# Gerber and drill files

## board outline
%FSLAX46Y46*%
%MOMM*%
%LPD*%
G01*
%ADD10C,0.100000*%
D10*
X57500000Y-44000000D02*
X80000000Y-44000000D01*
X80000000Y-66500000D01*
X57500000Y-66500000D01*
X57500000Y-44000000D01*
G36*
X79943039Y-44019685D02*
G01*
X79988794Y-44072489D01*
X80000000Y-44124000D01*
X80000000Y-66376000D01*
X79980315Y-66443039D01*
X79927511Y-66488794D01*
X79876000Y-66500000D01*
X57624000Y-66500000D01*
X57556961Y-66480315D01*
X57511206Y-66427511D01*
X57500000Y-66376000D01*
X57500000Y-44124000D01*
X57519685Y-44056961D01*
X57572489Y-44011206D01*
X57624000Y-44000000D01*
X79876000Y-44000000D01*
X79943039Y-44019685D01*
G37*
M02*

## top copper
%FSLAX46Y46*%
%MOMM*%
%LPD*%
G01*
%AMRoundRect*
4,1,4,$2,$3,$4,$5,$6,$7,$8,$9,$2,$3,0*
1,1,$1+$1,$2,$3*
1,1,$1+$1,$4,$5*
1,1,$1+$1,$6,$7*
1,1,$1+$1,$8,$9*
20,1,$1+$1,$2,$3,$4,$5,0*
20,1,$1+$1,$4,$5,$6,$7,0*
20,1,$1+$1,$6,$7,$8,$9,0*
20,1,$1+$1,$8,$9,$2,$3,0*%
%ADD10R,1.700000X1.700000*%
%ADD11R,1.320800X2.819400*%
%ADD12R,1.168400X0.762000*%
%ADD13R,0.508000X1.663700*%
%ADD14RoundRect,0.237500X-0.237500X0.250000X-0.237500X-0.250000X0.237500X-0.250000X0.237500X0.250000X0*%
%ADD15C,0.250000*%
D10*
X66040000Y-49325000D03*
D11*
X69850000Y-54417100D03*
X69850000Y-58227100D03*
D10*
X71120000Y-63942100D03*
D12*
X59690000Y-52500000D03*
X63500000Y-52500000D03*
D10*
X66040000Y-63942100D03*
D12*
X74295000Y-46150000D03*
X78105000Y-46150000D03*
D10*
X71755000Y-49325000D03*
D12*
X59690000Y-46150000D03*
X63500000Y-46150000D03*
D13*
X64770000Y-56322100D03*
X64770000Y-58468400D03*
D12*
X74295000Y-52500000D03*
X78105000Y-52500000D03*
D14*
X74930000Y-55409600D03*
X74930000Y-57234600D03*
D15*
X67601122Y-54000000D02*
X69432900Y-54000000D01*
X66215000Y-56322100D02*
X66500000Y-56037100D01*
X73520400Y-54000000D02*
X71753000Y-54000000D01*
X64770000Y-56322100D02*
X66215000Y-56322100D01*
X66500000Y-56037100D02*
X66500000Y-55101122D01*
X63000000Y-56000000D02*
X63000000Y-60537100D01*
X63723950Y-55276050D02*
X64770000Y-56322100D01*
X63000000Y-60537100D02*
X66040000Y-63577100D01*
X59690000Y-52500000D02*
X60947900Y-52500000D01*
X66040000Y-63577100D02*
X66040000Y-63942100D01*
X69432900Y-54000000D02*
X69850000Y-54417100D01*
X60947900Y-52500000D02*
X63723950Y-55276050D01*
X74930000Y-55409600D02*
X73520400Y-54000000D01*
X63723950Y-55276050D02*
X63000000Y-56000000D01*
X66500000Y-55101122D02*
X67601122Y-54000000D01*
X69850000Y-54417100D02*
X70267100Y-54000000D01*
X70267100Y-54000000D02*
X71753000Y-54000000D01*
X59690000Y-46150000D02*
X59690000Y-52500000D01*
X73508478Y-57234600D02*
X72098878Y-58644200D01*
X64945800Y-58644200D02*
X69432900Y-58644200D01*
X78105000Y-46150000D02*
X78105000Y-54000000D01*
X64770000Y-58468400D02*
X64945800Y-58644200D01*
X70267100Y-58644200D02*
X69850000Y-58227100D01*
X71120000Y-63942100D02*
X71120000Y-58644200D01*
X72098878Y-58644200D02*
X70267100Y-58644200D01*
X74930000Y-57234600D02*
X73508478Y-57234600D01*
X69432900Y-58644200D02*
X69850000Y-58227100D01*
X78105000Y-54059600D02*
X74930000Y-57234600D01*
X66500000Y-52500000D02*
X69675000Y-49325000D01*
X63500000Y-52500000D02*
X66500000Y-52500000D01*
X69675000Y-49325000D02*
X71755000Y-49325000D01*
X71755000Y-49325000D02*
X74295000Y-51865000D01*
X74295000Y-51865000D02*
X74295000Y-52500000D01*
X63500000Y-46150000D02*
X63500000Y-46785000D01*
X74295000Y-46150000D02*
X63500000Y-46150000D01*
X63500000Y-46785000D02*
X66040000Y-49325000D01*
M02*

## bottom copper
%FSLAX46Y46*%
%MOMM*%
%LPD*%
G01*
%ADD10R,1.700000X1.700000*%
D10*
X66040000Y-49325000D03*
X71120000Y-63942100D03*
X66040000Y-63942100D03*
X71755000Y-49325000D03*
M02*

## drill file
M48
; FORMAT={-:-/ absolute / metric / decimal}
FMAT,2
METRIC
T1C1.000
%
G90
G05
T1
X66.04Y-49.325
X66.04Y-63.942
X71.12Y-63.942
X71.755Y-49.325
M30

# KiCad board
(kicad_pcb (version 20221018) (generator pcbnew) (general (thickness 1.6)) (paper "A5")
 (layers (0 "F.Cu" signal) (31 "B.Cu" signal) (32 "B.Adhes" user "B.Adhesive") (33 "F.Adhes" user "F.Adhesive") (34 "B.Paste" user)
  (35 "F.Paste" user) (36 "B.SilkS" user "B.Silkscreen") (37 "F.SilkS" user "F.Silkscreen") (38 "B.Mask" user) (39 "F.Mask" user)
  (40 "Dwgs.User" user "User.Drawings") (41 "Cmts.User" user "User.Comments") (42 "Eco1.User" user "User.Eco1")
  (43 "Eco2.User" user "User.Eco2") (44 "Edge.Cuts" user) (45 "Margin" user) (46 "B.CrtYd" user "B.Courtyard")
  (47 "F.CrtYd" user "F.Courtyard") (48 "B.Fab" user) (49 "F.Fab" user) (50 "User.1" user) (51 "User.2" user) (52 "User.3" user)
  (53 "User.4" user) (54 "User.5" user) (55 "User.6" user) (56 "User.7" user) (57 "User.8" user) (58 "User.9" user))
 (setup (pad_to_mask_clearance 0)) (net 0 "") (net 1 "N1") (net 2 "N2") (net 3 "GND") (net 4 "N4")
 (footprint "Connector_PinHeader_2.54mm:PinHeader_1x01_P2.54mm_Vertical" (layer "F.Cu") (at 66.04 49.325)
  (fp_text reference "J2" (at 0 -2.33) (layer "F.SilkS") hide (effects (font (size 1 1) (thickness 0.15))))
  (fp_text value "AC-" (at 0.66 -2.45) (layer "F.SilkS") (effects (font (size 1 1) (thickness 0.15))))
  (pad "1" thru_hole rect (at 0 0) (size 1.7 1.7) (drill 1) (layers "*.Cu" "*.Mask") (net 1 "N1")))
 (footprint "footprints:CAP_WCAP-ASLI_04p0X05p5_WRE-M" (layer "F.Cu") (at 69.85 56.3221 -90)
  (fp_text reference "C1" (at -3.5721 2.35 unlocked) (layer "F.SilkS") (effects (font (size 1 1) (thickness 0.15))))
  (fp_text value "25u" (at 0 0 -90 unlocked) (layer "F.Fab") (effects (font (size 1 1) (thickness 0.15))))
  (pad "1" smd rect (at -1.905 0 270) (size 2.8194 1.3208) (layers "F.Cu" "F.Paste" "F.Mask") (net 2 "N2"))
  (pad "2" smd rect (at 1.905 0 270) (size 2.8194 1.3208) (layers "F.Cu" "F.Paste" "F.Mask") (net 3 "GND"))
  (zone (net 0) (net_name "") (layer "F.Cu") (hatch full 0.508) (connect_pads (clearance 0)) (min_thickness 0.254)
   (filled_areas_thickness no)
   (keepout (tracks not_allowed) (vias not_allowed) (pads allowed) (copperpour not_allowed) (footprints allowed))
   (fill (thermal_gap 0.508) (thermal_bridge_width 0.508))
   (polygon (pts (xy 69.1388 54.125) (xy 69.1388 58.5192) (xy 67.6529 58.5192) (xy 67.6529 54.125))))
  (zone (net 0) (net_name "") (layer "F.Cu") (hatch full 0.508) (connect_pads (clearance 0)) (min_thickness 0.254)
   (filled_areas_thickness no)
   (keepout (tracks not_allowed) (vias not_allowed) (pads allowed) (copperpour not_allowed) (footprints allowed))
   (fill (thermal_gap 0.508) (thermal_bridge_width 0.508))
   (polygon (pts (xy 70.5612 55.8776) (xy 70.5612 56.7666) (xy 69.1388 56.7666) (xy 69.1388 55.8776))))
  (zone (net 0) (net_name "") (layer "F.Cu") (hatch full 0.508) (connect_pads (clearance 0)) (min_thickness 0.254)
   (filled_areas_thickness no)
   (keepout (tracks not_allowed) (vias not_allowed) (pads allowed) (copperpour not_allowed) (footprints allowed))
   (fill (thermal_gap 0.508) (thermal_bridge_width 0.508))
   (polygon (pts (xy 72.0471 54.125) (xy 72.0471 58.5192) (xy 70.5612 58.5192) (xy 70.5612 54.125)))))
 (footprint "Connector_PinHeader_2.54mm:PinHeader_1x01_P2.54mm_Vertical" (layer "F.Cu") (at 71.12 63.9421 90)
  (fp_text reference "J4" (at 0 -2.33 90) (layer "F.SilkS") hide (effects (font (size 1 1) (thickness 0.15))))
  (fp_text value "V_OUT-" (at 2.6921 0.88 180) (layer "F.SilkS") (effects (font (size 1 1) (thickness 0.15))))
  (pad "1" thru_hole rect (at 0 0 90) (size 1.7 1.7) (drill 1) (layers "*.Cu" "*.Mask") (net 3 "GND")))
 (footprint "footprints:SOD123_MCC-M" (layer "F.Cu") (at 61.595 52.5)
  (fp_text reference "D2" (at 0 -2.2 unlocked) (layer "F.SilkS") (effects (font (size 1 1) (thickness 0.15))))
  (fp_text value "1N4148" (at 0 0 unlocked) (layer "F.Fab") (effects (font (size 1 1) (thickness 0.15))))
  (pad "1" smd rect (at -1.905 0) (size 1.1684 0.762) (layers "F.Cu" "F.Paste" "F.Mask") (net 2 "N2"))
  (pad "2" smd rect (at 1.905 0) (size 1.1684 0.762) (layers "F.Cu" "F.Paste" "F.Mask") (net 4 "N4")))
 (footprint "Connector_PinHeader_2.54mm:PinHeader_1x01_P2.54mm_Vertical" (layer "F.Cu") (at 66.04 63.9421 180)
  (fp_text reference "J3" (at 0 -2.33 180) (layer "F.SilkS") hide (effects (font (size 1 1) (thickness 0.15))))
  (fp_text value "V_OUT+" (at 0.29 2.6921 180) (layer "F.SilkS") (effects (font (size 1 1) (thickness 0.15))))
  (pad "1" thru_hole rect (at 0 0 180) (size 1.7 1.7) (drill 1) (layers "*.Cu" "*.Mask") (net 2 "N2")))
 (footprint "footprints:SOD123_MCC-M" (layer "F.Cu") (at 76.2 46.15)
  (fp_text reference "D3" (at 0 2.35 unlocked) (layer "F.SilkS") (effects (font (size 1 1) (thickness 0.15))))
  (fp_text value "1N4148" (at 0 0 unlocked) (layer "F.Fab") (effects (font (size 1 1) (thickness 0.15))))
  (pad "1" smd rect (at -1.905 0) (size 1.1684 0.762) (layers "F.Cu" "F.Paste" "F.Mask") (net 1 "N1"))
  (pad "2" smd rect (at 1.905 0) (size 1.1684 0.762) (layers "F.Cu" "F.Paste" "F.Mask") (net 3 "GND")))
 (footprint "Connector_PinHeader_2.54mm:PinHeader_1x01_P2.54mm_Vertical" (layer "F.Cu") (at 71.755 49.325)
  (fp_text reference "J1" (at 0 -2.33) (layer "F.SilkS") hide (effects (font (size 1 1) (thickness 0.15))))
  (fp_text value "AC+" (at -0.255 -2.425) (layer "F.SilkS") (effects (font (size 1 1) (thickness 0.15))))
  (pad "1" thru_hole rect (at 0 0) (size 1.7 1.7) (drill 1) (layers "*.Cu" "*.Mask") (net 4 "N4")))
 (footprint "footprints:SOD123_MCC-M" (layer "F.Cu") (at 61.595 46.15)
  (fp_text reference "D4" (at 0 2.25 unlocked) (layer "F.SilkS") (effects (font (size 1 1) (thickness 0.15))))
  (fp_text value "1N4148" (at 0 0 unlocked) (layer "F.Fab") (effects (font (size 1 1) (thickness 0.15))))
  (pad "1" smd rect (at -1.905 0) (size 1.1684 0.762) (layers "F.Cu" "F.Paste" "F.Mask") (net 2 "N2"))
  (pad "2" smd rect (at 1.905 0) (size 1.1684 0.762) (layers "F.Cu" "F.Paste" "F.Mask") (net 1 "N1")))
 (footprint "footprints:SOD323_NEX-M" (layer "F.Cu") (at 64.77 57.39525 -90)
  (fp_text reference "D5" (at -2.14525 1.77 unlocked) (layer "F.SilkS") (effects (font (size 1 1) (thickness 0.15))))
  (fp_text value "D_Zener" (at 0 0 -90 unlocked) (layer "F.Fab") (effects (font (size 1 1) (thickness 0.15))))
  (pad "1" smd rect (at -1.07315 0 270) (size 1.6637 0.508) (layers "F.Cu" "F.Paste" "F.Mask") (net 2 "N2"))
  (pad "2" smd rect (at 1.07315 0 270) (size 1.6637 0.508) (layers "F.Cu" "F.Paste" "F.Mask") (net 3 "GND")))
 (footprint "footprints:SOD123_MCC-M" (layer "F.Cu") (at 76.2 52.5)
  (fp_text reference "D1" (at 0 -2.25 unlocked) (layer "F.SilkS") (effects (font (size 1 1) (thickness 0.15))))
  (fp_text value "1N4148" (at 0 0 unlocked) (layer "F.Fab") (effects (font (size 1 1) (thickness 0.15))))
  (pad "1" smd rect (at -1.905 0) (size 1.1684 0.762) (layers "F.Cu" "F.Paste" "F.Mask") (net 4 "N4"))
  (pad "2" smd rect (at 1.905 0) (size 1.1684 0.762) (layers "F.Cu" "F.Paste" "F.Mask") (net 3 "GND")))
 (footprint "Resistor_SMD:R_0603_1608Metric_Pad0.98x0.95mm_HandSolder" (layer "F.Cu") (at 74.93 56.3221 -90)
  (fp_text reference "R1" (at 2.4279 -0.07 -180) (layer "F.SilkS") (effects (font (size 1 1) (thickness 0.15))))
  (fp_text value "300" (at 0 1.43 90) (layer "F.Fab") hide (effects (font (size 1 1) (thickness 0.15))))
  (pad "1" smd roundrect (at -0.9125 0 270) (size 0.975 0.95) (layers "F.Cu" "F.Paste" "F.Mask") (roundrect_rratio 0.25) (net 2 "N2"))
  (pad "2" smd roundrect (at 0.9125 0 270) (size 0.975 0.95) (layers "F.Cu" "F.Paste" "F.Mask") (roundrect_rratio 0.25) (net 3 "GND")))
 (gr_rect (start 57.5 44) (end 80 66.5) (stroke (width 0.1) (type default)) (fill none) (layer "Edge.Cuts"))
 (segment (start 67.601122 54) (end 69.4329 54) (width 0.25) (layer "F.Cu") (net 2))
 (segment (start 66.215 56.3221) (end 66.5 56.0371) (width 0.25) (layer "F.Cu") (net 2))
 (segment (start 73.5204 54) (end 71.753 54) (width 0.25) (layer "F.Cu") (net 2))
 (segment (start 64.77 56.3221) (end 66.215 56.3221) (width 0.25) (layer "F.Cu") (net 2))
 (segment (start 66.5 56.0371) (end 66.5 55.101122) (width 0.25) (layer "F.Cu") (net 2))
 (segment (start 63 56) (end 63 60.5371) (width 0.25) (layer "F.Cu") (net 2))
 (segment (start 63.72395 55.27605) (end 64.77 56.3221) (width 0.25) (layer "F.Cu") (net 2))
 (segment (start 63 60.5371) (end 66.04 63.5771) (width 0.25) (layer "F.Cu") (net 2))
 (segment (start 59.69 52.5) (end 60.9479 52.5) (width 0.25) (layer "F.Cu") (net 2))
 (segment (start 66.04 63.5771) (end 66.04 63.9421) (width 0.25) (layer "F.Cu") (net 2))
 (segment (start 69.4329 54) (end 69.85 54.4171) (width 0.25) (layer "F.Cu") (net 2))
 (segment (start 60.9479 52.5) (end 63.72395 55.27605) (width 0.25) (layer "F.Cu") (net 2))
 (segment (start 74.93 55.4096) (end 73.5204 54) (width 0.25) (layer "F.Cu") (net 2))
 (segment (start 63.72395 55.27605) (end 63 56) (width 0.25) (layer "F.Cu") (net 2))
 (segment (start 66.5 55.101122) (end 67.601122 54) (width 0.25) (layer "F.Cu") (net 2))
 (segment (start 69.85 54.4171) (end 70.2671 54) (width 0.25) (layer "F.Cu") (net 2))
 (segment (start 70.2671 54) (end 71.753 54) (width 0.25) (layer "F.Cu") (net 2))
 (segment (start 59.69 46.15) (end 59.69 52.5) (width 0.25) (layer "F.Cu") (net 2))
 (segment (start 73.508478 57.2346) (end 72.098878 58.6442) (width 0.25) (layer "F.Cu") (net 3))
 (segment (start 64.9458 58.6442) (end 69.4329 58.6442) (width 0.25) (layer "F.Cu") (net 3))
 (segment (start 78.105 46.15) (end 78.105 54) (width 0.25) (layer "F.Cu") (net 3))
 (segment (start 64.77 58.4684) (end 64.9458 58.6442) (width 0.25) (layer "F.Cu") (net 3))
 (segment (start 70.2671 58.6442) (end 69.85 58.2271) (width 0.25) (layer "F.Cu") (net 3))
 (segment (start 71.12 63.9421) (end 71.12 58.6442) (width 0.25) (layer "F.Cu") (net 3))
 (segment (start 72.098878 58.6442) (end 70.2671 58.6442) (width 0.25) (layer "F.Cu") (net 3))
 (segment (start 74.93 57.2346) (end 73.508478 57.2346) (width 0.25) (layer "F.Cu") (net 3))
 (segment (start 69.4329 58.6442) (end 69.85 58.2271) (width 0.25) (layer "F.Cu") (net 3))
 (segment (start 78.105 54.0596) (end 74.93 57.2346) (width 0.25) (layer "F.Cu") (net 3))
 (segment (start 66.5 52.5) (end 69.675 49.325) (width 0.25) (layer "F.Cu") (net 4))
 (segment (start 63.5 52.5) (end 66.5 52.5) (width 0.25) (layer "F.Cu") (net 4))
 (segment (start 69.675 49.325) (end 71.755 49.325) (width 0.25) (layer "F.Cu") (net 4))
 (segment (start 71.755 49.325) (end 74.295 51.865) (width 0.25) (layer "F.Cu") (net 4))
 (segment (start 74.295 51.865) (end 74.295 52.5) (width 0.25) (layer "F.Cu") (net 4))
 (segment (start 63.5 46.15) (end 63.5 46.785) (width 0.25) (layer "F.Cu") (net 1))
 (segment (start 74.295 46.15) (end 63.5 46.15) (width 0.25) (layer "F.Cu") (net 1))
 (segment (start 63.5 46.785) (end 66.04 49.325) (width 0.25) (layer "F.Cu") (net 1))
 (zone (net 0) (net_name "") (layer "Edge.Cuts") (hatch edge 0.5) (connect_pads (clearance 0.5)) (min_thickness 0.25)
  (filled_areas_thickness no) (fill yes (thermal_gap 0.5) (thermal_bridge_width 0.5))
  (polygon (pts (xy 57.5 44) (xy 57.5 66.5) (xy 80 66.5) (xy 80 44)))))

